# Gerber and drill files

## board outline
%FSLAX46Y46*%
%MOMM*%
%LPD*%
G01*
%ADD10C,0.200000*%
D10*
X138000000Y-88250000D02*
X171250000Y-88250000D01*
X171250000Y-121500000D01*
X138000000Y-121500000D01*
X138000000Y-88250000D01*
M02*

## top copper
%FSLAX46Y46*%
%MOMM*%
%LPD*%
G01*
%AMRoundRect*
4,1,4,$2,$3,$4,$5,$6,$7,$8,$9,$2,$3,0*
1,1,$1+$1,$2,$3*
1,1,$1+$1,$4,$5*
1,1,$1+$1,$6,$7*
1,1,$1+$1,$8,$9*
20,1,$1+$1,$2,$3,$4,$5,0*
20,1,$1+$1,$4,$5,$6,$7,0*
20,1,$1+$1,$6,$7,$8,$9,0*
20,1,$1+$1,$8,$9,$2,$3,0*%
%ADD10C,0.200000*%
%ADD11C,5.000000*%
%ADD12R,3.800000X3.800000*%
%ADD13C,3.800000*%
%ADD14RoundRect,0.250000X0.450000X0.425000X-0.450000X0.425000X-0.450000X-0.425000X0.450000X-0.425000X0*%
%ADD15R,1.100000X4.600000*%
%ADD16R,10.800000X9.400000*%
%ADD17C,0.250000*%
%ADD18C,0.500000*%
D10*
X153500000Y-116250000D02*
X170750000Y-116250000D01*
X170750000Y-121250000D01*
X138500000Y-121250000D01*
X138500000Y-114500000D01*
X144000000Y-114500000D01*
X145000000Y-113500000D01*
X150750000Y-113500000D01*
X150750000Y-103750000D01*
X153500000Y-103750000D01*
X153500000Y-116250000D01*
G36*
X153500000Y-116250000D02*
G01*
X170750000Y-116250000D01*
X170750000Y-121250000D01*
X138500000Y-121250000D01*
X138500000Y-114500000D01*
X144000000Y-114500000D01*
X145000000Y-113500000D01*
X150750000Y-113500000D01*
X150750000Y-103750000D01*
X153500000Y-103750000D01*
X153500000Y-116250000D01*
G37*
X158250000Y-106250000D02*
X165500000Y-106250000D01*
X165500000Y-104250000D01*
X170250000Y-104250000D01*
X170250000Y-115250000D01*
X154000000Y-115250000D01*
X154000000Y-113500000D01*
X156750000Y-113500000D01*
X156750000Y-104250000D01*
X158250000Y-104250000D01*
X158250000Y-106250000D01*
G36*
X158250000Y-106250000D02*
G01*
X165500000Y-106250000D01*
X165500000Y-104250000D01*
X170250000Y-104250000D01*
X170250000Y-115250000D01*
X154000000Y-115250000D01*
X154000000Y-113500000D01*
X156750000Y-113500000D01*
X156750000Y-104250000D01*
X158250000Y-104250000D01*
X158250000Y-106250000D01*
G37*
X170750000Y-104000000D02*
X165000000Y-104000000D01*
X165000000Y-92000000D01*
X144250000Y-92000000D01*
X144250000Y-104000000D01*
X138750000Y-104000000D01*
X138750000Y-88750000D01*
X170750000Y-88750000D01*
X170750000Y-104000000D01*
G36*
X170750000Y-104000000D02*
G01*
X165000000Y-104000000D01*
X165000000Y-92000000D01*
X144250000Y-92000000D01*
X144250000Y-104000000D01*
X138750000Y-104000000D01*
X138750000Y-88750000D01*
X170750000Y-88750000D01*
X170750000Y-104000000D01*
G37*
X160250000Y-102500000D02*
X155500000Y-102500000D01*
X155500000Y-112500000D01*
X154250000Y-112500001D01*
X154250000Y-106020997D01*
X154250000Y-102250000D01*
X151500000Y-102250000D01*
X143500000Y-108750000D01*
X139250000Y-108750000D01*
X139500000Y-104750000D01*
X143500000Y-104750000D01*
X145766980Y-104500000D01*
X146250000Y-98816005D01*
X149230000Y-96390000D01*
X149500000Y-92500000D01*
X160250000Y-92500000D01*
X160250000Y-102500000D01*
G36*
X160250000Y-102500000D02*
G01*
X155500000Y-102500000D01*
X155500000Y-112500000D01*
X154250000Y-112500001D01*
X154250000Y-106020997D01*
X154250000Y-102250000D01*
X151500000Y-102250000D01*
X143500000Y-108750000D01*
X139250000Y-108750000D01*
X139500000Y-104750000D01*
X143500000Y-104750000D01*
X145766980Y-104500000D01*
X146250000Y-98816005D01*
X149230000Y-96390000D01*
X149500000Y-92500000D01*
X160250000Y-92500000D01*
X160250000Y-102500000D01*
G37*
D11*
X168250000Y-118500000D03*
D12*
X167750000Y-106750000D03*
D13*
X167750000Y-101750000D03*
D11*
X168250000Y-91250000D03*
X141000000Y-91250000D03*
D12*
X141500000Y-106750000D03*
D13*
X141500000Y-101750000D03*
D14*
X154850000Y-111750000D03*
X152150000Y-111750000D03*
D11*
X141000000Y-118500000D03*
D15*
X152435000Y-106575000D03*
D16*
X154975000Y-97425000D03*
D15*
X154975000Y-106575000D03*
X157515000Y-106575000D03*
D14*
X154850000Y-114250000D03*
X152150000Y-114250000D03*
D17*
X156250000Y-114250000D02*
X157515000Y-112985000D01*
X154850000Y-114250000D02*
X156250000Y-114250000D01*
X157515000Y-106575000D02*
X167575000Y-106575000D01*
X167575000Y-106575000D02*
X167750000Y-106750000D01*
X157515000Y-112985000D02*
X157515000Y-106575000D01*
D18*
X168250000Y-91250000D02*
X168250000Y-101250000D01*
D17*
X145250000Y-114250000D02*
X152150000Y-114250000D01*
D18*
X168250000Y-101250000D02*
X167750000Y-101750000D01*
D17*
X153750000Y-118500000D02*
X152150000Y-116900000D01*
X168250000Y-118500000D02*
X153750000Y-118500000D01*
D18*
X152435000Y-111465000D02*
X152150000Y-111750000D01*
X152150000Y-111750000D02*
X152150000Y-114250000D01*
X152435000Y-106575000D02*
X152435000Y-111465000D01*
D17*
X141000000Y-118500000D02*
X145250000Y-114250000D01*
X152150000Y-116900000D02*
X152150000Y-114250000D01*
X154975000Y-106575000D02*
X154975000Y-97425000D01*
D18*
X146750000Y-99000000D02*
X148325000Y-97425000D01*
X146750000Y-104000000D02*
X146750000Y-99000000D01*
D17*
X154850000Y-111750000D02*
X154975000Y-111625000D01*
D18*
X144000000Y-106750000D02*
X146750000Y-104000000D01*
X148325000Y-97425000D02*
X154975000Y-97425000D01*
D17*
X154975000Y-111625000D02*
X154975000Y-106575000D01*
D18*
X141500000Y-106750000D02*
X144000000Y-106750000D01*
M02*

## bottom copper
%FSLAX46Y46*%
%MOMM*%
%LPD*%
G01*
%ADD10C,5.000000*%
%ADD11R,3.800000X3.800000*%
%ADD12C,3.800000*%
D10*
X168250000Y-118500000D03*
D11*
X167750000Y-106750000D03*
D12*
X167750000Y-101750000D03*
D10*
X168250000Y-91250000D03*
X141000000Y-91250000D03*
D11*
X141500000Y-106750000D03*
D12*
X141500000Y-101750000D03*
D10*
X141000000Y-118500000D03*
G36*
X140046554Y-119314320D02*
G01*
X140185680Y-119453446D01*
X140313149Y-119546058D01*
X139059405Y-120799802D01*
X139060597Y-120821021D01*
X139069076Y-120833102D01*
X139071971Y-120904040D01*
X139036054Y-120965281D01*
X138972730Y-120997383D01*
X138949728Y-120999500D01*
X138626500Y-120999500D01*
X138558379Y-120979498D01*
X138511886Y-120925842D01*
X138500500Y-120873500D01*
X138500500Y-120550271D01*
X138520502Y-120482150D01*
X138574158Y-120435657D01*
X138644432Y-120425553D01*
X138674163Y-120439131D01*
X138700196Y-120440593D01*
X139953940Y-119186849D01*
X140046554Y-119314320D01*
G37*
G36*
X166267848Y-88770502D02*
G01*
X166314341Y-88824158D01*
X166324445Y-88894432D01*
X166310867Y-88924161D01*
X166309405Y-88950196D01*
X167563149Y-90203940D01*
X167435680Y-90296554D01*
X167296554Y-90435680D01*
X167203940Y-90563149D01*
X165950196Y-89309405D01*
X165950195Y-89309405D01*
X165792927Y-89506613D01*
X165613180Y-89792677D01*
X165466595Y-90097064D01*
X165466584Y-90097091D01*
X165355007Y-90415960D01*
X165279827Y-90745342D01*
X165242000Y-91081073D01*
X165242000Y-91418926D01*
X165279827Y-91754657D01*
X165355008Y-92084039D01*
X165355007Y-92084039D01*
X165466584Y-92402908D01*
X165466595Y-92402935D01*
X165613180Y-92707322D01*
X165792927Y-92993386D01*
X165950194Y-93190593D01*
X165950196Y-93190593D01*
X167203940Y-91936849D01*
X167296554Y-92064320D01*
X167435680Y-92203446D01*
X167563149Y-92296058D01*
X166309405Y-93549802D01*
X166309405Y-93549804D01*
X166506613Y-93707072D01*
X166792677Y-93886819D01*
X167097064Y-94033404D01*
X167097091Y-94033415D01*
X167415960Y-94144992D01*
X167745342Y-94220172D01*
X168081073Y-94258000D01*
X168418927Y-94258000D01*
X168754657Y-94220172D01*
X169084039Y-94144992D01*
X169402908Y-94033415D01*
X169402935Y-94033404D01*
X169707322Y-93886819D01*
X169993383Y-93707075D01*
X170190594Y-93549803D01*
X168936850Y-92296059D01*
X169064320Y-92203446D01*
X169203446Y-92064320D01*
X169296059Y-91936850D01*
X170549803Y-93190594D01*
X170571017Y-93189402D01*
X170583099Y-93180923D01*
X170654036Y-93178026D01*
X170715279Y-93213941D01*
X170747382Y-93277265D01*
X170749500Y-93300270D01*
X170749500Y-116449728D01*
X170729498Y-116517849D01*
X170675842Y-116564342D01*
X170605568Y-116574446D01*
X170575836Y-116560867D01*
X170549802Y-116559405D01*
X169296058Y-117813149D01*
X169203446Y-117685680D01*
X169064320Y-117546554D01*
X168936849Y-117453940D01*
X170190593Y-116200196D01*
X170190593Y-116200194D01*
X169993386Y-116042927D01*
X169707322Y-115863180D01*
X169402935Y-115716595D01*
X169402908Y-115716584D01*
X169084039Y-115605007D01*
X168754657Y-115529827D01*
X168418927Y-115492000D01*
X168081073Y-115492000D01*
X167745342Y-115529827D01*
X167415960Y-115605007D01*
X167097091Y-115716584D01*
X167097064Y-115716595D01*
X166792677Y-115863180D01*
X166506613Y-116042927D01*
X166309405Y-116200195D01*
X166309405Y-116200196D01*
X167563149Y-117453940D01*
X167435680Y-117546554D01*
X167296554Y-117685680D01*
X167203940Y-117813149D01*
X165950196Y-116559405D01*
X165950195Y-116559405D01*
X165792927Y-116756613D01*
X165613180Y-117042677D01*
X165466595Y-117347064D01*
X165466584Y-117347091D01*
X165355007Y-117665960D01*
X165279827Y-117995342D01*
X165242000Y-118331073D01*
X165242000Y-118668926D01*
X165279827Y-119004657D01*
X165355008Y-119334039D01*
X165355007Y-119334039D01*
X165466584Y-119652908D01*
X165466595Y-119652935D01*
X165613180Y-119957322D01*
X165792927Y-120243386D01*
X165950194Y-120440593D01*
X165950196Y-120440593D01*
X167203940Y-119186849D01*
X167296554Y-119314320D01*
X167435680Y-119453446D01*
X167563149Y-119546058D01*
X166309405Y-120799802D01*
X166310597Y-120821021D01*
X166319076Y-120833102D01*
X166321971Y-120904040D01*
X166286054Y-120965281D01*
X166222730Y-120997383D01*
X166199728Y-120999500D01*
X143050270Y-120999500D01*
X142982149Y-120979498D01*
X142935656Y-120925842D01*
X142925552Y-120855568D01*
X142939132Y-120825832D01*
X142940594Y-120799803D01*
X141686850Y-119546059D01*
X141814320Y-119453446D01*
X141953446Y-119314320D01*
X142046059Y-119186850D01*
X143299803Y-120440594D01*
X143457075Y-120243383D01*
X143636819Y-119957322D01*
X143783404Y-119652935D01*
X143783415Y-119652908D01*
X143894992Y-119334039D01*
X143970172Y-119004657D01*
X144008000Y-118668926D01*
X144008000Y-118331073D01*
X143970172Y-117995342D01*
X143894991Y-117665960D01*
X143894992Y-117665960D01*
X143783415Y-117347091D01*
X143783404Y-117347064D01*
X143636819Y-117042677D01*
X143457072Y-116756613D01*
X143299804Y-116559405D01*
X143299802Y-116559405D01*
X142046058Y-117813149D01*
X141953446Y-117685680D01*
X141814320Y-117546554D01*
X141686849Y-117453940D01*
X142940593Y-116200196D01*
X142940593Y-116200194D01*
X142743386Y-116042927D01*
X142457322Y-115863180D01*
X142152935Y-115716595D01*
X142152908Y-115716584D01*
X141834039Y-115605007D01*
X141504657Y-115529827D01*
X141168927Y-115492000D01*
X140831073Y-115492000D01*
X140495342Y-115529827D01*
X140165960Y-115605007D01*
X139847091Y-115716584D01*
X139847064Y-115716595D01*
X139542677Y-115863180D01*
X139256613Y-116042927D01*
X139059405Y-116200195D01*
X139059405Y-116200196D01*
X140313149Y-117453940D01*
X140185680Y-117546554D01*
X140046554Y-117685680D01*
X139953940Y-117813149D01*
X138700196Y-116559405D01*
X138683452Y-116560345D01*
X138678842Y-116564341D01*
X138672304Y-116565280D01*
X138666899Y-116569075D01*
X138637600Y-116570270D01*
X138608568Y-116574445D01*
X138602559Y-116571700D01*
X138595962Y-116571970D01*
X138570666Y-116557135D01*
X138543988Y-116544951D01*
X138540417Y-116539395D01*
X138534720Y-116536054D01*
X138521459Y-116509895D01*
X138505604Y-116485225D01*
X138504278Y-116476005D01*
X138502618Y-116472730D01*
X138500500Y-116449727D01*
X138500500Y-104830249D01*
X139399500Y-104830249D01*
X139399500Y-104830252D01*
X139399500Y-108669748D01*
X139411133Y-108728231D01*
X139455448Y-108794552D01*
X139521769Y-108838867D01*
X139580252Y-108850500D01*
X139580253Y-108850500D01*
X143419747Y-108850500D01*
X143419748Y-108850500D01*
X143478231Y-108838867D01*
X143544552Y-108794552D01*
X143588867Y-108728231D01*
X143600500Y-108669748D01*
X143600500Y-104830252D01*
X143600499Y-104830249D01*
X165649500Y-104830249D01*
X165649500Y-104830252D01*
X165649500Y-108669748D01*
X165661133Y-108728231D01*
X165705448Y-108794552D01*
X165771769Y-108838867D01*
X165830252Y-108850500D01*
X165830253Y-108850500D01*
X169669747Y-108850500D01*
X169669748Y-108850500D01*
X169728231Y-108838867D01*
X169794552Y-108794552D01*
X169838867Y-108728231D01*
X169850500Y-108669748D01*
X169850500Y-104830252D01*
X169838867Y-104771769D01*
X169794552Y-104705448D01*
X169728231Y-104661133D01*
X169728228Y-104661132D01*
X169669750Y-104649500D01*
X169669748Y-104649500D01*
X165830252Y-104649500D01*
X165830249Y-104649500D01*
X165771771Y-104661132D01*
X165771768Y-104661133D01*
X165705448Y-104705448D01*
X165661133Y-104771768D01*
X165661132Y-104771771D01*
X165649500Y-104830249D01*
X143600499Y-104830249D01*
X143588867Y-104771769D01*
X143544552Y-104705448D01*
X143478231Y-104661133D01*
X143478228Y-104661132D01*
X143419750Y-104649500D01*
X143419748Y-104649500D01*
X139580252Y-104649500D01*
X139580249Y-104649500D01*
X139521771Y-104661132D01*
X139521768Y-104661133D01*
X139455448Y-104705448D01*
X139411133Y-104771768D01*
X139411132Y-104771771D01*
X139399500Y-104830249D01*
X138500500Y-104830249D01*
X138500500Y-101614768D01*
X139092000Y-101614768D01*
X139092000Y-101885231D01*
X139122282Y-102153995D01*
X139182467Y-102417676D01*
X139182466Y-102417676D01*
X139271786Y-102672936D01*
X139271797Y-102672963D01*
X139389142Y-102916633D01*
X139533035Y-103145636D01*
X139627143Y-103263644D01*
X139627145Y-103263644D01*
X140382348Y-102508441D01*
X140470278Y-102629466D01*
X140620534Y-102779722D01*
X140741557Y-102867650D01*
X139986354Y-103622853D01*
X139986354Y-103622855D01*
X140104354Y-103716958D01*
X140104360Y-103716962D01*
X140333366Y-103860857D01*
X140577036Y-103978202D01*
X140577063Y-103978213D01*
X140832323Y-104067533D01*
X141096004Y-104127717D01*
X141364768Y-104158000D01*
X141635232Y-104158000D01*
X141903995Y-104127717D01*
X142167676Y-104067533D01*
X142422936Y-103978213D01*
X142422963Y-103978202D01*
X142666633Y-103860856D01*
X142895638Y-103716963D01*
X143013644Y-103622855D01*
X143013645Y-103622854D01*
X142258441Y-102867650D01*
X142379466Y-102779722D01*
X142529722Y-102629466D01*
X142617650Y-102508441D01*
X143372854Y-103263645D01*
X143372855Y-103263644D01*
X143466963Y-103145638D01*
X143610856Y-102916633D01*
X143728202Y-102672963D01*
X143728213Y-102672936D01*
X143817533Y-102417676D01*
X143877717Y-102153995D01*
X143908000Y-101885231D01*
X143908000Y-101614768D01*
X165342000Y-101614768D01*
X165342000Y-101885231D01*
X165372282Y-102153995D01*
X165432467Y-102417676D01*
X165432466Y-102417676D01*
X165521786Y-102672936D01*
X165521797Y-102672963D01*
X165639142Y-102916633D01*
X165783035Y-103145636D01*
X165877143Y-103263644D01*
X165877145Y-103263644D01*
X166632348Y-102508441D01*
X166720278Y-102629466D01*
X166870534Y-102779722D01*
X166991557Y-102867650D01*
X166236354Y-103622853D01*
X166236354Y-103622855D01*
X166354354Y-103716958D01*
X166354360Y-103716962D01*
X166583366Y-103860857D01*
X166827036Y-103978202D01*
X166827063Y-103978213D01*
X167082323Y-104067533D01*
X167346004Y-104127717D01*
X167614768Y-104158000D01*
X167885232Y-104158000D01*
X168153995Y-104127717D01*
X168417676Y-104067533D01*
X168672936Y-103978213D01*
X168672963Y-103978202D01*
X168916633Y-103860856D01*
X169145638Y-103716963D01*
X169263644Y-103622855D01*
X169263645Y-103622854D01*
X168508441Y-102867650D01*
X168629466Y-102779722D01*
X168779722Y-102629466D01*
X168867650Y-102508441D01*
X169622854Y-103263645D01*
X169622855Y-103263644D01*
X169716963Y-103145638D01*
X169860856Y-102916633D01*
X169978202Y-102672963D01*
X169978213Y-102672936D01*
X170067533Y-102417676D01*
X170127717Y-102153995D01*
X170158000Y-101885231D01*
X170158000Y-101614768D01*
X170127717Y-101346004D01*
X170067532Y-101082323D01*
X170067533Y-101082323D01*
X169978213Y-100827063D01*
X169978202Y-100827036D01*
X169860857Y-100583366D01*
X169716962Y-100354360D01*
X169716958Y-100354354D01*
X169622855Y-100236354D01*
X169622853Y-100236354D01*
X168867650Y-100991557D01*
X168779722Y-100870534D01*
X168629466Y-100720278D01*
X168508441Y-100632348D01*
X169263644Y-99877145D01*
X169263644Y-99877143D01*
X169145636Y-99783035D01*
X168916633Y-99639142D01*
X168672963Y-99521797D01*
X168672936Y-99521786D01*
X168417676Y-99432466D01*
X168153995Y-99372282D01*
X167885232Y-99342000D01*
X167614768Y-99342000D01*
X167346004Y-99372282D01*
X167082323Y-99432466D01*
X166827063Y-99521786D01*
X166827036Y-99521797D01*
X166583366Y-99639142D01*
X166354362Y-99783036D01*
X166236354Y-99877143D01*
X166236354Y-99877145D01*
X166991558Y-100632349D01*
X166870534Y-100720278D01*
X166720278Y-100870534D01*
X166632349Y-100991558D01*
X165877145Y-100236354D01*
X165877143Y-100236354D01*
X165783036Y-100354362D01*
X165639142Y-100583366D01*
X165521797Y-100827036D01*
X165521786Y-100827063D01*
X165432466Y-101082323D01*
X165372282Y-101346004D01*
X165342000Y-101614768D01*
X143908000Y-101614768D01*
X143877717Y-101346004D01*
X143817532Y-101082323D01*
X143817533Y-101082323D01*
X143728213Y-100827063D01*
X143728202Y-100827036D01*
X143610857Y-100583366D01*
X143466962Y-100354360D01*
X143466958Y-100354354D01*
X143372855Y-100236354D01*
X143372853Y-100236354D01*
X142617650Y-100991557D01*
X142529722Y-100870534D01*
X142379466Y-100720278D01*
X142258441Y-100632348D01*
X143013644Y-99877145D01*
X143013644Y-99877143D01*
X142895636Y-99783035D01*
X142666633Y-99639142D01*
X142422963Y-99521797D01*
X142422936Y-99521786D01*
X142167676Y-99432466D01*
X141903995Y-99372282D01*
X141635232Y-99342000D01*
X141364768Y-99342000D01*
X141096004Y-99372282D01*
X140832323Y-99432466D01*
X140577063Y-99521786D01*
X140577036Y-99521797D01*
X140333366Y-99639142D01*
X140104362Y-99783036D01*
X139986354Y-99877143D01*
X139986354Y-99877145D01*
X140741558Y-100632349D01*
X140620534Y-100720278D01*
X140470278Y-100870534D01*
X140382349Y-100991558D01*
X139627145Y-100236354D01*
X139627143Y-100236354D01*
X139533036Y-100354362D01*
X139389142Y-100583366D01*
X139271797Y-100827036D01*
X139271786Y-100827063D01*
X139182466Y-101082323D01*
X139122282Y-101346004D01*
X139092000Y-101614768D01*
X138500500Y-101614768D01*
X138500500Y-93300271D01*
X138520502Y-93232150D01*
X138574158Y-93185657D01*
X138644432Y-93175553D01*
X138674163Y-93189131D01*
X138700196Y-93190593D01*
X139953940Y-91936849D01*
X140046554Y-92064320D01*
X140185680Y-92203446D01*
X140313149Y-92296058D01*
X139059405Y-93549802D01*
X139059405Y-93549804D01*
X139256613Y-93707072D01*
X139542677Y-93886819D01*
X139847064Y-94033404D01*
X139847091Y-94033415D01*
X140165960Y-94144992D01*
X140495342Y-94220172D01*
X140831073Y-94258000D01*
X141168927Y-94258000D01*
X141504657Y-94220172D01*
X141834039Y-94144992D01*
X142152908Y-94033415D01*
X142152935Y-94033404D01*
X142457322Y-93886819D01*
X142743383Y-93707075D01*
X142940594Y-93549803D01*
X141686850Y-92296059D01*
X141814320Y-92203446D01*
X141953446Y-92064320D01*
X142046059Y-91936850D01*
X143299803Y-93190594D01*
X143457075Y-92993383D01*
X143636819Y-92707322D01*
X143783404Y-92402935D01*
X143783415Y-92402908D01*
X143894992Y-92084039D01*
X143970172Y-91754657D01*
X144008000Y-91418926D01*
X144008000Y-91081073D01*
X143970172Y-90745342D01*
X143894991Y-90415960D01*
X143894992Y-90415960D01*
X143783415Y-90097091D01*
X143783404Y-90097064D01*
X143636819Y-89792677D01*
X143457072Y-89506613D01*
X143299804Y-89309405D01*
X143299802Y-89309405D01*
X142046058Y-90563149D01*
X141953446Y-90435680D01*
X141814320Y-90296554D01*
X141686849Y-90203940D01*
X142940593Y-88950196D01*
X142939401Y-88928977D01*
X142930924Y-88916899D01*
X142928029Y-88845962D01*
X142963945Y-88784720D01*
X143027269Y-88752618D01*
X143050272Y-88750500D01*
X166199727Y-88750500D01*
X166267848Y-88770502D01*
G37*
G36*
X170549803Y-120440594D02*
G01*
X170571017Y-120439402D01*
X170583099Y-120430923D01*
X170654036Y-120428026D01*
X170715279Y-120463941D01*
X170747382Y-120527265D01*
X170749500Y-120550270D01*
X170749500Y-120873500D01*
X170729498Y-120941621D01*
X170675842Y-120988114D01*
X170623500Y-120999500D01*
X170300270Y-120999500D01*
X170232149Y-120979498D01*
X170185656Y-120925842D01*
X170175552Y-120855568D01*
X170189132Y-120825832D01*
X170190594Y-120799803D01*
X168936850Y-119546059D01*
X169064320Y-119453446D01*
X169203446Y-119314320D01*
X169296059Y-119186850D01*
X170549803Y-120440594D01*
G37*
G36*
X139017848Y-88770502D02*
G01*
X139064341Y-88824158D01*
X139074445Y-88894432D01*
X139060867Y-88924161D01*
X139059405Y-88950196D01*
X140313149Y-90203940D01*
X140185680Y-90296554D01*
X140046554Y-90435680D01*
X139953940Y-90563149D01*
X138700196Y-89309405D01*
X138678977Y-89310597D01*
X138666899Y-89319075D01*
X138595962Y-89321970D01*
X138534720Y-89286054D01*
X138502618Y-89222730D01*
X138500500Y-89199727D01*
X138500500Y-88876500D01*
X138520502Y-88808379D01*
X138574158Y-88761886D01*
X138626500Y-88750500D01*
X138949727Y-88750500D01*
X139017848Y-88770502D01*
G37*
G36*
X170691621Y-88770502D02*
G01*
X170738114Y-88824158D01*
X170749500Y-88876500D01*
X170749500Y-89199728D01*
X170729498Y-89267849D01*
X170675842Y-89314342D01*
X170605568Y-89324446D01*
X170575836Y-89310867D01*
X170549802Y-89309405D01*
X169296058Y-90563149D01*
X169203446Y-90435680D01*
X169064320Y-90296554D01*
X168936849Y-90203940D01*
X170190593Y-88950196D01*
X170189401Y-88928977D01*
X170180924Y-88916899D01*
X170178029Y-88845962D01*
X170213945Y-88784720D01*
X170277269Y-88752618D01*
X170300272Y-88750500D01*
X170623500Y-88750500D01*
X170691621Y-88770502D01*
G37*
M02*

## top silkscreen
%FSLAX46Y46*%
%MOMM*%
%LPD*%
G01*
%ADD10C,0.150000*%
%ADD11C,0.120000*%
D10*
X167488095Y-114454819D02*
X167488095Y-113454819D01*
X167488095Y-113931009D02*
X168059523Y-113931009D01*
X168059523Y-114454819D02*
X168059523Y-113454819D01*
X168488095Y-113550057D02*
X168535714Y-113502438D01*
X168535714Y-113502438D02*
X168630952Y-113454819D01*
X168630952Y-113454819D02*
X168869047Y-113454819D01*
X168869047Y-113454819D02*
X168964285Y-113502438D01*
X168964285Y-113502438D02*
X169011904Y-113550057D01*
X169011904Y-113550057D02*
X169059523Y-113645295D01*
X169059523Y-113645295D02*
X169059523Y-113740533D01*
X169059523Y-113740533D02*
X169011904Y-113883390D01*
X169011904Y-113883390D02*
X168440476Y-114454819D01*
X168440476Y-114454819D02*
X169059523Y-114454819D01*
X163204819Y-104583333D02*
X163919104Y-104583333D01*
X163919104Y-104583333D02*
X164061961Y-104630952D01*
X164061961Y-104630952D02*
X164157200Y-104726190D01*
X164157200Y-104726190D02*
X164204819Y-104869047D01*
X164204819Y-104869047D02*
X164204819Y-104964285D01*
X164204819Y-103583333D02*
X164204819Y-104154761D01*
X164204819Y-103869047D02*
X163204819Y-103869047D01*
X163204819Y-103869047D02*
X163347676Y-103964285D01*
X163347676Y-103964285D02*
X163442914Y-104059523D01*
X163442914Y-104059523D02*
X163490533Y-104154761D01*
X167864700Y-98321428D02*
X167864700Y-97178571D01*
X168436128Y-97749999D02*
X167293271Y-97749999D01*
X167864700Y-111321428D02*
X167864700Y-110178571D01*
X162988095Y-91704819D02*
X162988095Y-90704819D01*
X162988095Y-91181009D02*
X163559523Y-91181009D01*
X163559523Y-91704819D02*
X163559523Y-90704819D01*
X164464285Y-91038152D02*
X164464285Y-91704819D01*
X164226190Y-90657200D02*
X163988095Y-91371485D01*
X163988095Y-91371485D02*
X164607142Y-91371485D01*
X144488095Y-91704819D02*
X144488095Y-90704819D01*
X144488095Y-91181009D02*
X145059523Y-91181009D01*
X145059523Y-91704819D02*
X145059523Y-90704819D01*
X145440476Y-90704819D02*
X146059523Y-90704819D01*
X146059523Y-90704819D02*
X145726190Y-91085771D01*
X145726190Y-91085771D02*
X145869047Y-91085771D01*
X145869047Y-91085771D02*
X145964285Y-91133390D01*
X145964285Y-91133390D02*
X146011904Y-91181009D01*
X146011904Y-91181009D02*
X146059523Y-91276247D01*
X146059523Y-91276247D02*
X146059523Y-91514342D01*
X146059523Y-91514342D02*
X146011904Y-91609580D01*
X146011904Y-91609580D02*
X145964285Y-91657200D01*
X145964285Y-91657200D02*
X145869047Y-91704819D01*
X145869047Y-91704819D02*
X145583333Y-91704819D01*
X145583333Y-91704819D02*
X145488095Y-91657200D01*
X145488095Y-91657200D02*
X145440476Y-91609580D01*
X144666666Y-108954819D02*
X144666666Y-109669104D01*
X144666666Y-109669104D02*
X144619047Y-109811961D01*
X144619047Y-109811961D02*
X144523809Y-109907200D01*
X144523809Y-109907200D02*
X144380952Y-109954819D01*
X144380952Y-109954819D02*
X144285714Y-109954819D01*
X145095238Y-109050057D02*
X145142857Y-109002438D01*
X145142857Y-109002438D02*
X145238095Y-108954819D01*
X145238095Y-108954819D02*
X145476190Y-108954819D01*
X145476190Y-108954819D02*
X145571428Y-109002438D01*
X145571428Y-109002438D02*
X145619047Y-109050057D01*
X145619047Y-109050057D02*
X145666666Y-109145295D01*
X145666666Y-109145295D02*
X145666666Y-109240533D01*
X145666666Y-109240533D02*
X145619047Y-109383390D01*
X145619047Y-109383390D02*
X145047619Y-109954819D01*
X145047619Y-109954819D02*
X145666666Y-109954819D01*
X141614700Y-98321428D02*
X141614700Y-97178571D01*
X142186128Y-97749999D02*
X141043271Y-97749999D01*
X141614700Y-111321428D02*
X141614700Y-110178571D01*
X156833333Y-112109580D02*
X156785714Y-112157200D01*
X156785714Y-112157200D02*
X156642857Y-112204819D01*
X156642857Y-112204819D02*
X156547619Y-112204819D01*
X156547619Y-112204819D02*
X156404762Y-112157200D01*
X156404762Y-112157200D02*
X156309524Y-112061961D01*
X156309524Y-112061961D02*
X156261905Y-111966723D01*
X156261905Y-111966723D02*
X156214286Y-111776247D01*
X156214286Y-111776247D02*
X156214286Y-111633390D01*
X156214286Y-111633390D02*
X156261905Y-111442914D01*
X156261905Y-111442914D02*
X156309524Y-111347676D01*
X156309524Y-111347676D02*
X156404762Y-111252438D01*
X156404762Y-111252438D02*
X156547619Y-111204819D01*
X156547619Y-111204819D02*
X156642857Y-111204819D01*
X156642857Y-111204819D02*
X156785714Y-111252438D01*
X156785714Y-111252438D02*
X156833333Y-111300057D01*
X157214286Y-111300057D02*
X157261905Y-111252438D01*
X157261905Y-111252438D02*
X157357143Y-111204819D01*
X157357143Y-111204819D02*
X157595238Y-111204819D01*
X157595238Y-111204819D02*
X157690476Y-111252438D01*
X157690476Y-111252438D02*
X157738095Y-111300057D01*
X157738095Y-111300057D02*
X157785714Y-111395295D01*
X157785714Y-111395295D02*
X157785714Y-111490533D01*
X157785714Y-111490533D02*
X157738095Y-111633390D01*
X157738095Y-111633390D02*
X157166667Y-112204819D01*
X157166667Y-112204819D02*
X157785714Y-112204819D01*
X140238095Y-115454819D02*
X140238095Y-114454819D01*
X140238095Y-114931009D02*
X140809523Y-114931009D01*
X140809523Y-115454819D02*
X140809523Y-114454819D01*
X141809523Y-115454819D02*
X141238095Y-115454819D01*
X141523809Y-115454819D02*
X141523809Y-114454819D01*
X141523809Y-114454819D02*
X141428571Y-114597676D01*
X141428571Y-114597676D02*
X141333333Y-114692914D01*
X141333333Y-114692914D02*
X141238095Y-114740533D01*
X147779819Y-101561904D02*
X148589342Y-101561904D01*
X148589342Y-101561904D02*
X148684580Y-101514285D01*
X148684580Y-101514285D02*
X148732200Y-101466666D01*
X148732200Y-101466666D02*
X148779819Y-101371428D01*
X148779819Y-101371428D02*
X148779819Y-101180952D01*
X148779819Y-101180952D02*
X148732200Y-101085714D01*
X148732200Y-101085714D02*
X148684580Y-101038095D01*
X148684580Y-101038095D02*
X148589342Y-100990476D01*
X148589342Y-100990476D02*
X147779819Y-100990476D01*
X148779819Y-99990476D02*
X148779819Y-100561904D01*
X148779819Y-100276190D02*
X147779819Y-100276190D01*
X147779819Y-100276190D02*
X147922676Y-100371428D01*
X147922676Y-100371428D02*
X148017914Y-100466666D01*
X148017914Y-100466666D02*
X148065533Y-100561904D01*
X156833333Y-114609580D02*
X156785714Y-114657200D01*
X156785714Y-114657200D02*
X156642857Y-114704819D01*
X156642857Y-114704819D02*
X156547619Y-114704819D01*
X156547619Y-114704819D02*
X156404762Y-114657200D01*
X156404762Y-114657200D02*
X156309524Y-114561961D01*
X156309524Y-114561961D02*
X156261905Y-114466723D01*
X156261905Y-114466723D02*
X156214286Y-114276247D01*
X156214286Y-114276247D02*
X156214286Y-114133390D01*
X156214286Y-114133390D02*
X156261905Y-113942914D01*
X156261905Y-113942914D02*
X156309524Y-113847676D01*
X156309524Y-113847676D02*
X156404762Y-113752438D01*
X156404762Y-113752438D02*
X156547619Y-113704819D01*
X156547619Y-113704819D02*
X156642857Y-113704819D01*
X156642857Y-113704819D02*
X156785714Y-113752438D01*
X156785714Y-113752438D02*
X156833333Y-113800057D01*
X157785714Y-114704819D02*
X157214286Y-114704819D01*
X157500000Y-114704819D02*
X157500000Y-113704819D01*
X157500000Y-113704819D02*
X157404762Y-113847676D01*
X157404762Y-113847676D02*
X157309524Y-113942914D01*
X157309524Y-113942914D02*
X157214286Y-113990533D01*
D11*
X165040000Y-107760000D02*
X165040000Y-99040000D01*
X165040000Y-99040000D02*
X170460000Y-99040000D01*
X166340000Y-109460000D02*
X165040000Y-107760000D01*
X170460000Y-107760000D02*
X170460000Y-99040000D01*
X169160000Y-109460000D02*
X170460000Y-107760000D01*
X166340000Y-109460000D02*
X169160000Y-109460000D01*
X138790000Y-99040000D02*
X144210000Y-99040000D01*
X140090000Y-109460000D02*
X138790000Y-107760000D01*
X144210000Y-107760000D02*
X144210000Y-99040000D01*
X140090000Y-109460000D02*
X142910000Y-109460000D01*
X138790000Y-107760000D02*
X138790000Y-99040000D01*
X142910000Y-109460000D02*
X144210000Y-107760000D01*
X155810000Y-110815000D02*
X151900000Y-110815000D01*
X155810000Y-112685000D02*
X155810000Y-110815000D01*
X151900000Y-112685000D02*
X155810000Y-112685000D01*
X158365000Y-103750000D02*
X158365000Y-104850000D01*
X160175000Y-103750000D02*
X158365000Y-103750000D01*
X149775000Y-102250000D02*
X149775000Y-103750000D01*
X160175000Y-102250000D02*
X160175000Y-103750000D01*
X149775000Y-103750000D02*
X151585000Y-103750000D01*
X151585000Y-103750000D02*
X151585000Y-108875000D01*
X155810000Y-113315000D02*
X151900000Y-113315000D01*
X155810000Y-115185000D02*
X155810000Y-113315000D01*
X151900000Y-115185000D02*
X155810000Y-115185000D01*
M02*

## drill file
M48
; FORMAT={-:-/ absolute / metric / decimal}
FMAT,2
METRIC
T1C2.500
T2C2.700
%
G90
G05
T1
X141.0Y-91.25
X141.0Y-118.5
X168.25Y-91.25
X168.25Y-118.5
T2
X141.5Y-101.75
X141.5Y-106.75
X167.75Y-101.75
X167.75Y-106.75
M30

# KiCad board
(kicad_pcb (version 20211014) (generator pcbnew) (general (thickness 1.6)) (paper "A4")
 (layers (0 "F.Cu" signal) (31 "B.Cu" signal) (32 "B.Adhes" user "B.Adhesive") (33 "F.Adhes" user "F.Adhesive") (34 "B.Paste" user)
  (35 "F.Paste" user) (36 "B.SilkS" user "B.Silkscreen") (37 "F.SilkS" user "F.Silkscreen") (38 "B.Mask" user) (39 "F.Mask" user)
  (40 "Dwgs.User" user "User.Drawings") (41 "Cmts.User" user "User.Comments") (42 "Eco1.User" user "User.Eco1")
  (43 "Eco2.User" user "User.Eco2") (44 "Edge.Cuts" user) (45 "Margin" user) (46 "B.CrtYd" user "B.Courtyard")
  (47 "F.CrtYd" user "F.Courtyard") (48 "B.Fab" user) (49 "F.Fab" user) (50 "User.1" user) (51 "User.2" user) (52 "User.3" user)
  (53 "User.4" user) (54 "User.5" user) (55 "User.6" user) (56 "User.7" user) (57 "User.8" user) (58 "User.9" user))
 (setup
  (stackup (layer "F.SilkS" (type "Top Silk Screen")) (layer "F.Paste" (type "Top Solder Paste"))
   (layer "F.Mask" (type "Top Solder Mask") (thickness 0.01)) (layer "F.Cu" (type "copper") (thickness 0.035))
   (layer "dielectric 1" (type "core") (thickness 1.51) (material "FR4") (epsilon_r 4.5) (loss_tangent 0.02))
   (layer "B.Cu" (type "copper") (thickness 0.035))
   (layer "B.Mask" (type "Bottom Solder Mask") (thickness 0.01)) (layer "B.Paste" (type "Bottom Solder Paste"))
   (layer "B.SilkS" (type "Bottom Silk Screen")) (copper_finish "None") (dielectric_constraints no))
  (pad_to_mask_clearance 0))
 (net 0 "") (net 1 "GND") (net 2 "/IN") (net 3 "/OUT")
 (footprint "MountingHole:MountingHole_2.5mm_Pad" (layer "F.Cu") (at 168.25 118.5)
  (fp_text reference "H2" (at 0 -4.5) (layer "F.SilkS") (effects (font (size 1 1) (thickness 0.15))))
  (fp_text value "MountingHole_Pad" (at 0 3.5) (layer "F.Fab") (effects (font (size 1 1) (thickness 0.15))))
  (pad "1" thru_hole circle (at 0 0) (size 5 5) (drill 2.5) (layers *.Cu *.Mask) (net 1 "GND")))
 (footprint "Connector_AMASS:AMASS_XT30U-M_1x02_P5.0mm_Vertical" (layer "F.Cu") (at 167.75 106.75 90)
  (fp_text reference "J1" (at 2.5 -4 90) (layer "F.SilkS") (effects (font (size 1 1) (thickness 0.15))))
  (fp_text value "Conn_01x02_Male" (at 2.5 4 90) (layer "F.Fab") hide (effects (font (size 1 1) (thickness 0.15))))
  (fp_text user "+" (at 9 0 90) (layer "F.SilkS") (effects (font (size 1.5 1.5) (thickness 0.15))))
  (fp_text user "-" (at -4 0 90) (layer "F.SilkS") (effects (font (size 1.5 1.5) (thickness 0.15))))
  (fp_line (start -1.01 -2.71) (end 7.71 -2.71) (layer "F.SilkS") (width 0.12))
  (fp_line (start 7.71 -2.71) (end 7.71 2.71) (layer "F.SilkS") (width 0.12))
  (fp_line (start -2.71 -1.41) (end -1.01 -2.71) (layer "F.SilkS") (width 0.12))
  (fp_line (start -1.01 2.71) (end 7.71 2.71) (layer "F.SilkS") (width 0.12))
  (fp_line (start -2.71 1.41) (end -1.01 2.71) (layer "F.SilkS") (width 0.12))
  (fp_line (start -2.71 -1.41) (end -2.71 1.41) (layer "F.SilkS") (width 0.12))
  (pad "1" thru_hole rect (at 0 0 90) (size 3.8 3.8) (drill 2.7) (layers *.Cu *.Mask) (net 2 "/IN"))
  (pad "2" thru_hole circle (at 5 0 90) (size 3.8 3.8) (drill 2.7) (layers *.Cu *.Mask) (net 1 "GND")))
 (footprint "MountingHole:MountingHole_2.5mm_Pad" (layer "F.Cu") (at 168.25 91.25)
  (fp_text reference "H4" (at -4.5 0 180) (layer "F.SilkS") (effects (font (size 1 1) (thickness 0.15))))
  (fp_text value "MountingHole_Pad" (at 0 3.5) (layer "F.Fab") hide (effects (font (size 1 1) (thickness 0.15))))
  (pad "1" thru_hole circle (at 0 0) (size 5 5) (drill 2.5) (layers *.Cu *.Mask) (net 1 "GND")))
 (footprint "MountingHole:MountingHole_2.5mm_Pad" (layer "F.Cu") (at 141 91.25)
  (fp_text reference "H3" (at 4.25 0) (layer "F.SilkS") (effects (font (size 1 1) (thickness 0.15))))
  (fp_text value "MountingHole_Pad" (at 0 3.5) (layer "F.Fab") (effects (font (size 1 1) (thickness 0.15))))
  (pad "1" thru_hole circle (at 0 0) (size 5 5) (drill 2.5) (layers *.Cu *.Mask) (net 1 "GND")))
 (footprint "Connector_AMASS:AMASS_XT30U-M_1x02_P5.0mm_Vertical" (layer "F.Cu") (at 141.5 106.75 90)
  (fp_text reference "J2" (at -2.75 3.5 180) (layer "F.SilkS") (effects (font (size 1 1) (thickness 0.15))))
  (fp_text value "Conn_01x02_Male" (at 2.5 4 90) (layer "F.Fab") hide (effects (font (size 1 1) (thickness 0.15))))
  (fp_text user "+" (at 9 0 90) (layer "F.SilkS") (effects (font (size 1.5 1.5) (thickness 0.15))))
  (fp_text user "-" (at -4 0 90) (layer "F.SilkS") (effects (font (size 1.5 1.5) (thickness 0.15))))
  (fp_line (start 7.71 -2.71) (end 7.71 2.71) (layer "F.SilkS") (width 0.12))
  (fp_line (start -2.71 -1.41) (end -1.01 -2.71) (layer "F.SilkS") (width 0.12))
  (fp_line (start -1.01 2.71) (end 7.71 2.71) (layer "F.SilkS") (width 0.12))
  (fp_line (start -2.71 -1.41) (end -2.71 1.41) (layer "F.SilkS") (width 0.12))
  (fp_line (start -1.01 -2.71) (end 7.71 -2.71) (layer "F.SilkS") (width 0.12))
  (fp_line (start -2.71 1.41) (end -1.01 2.71) (layer "F.SilkS") (width 0.12))
  (pad "1" thru_hole rect (at 0 0 90) (size 3.8 3.8) (drill 2.7) (layers *.Cu *.Mask) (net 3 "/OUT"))
  (pad "2" thru_hole circle (at 5 0 90) (size 3.8 3.8) (drill 2.7) (layers *.Cu *.Mask) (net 1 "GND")))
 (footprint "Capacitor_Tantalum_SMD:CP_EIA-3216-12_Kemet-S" (layer "F.Cu") (at 153.5 111.75 180)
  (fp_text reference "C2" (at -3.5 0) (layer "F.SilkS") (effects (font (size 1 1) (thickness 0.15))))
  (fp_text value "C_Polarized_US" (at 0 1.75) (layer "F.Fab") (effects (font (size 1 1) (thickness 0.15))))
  (fp_line (start -2.31 0.935) (end 1.6 0.935) (layer "F.SilkS") (width 0.12))
  (fp_line (start -2.31 -0.935) (end -2.31 0.935) (layer "F.SilkS") (width 0.12))
  (fp_line (start 1.6 -0.935) (end -2.31 -0.935) (layer "F.SilkS") (width 0.12))
  (pad "1" smd roundrect (at -1.35 0 180) (size 1.4 1.35) (layers "F.Cu" "F.Paste" "F.Mask") (roundrect_rratio 0.185185) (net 3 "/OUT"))
  (pad "2" smd roundrect (at 1.35 0 180) (size 1.4 1.35) (layers "F.Cu" "F.Paste" "F.Mask") (roundrect_rratio 0.185185) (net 1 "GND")))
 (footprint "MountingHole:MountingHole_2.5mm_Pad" (layer "F.Cu") (at 141 118.5)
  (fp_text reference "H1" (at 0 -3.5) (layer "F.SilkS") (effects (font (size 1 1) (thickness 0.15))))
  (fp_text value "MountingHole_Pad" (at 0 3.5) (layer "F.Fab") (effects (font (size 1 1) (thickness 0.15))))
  (pad "1" thru_hole circle (at 0 0) (size 5 5) (drill 2.5) (layers *.Cu *.Mask) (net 1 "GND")))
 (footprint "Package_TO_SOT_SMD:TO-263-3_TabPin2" (layer "F.Cu") (at 154.975 100.8 90)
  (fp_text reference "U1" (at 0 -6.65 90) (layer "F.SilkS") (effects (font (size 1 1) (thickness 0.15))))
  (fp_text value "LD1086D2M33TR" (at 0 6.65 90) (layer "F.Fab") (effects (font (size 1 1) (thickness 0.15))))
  (fp_line (start -2.95 3.39) (end -4.05 3.39) (layer "F.SilkS") (width 0.12))
  (fp_line (start -2.95 5.2) (end -2.95 3.39) (layer "F.SilkS") (width 0.12))
  (fp_line (start -1.45 -5.2) (end -2.95 -5.2) (layer "F.SilkS") (width 0.12))
  (fp_line (start -1.45 5.2) (end -2.95 5.2) (layer "F.SilkS") (width 0.12))
  (fp_line (start -2.95 -5.2) (end -2.95 -3.39) (layer "F.SilkS") (width 0.12))
  (fp_line (start -2.95 -3.39) (end -8.075 -3.39) (layer "F.SilkS") (width 0.12))
  (pad "" smd rect (at 5.8 -2.775 90) (size 4.55 5.25) (layers "F.Paste"))
  (pad "" smd rect (at 5.8 2.775 90) (size 4.55 5.25) (layers "F.Paste"))
  (pad "" smd rect (at 0.95 2.775 90) (size 4.55 5.25) (layers "F.Paste"))
  (pad "" smd rect (at 0.95 -2.775 90) (size 4.55 5.25) (layers "F.Paste"))
  (pad "1" smd rect (at -5.775 -2.54 90) (size 4.6 1.1) (layers "F.Cu" "F.Paste" "F.Mask") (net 1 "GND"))
  (pad "2" smd rect (at 3.375 0 90) (size 9.4 10.8) (layers "F.Cu" "F.Mask") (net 3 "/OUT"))
  (pad "2" smd rect (at -5.775 0 90) (size 4.6 1.1) (layers "F.Cu" "F.Paste" "F.Mask") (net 3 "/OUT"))
  (pad "3" smd rect (at -5.775 2.54 90) (size 4.6 1.1) (layers "F.Cu" "F.Paste" "F.Mask") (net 2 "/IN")))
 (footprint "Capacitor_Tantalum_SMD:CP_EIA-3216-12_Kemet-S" (layer "F.Cu") (at 153.5 114.25 180)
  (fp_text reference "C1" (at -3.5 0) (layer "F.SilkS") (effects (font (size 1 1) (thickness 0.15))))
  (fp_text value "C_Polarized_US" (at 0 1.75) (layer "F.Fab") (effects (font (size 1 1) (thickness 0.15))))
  (fp_line (start -2.31 0.935) (end 1.6 0.935) (layer "F.SilkS") (width 0.12))
  (fp_line (start -2.31 -0.935) (end -2.31 0.935) (layer "F.SilkS") (width 0.12))
  (fp_line (start 1.6 -0.935) (end -2.31 -0.935) (layer "F.SilkS") (width 0.12))
  (pad "1" smd roundrect (at -1.35 0 180) (size 1.4 1.35) (layers "F.Cu" "F.Paste" "F.Mask") (roundrect_rratio 0.185185) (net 2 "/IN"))
  (pad "2" smd roundrect (at 1.35 0 180) (size 1.4 1.35) (layers "F.Cu" "F.Paste" "F.Mask") (roundrect_rratio 0.185185) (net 1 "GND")))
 (gr_poly
  (pts (xy 153.5 116.25) (xy 170.75 116.25) (xy 170.75 121.25) (xy 138.5 121.25) (xy 138.5 114.5) (xy 144 114.5) (xy 145 113.5)
   (xy 150.75 113.5) (xy 150.75 103.75) (xy 153.5 103.75))
  (layer "F.Cu") (width 0.2) (fill solid))
 (gr_poly
  (pts (xy 158.25 106.25) (xy 165.5 106.25) (xy 165.5 104.25) (xy 170.25 104.25) (xy 170.25 115.25) (xy 154 115.25) (xy 154 113.5)
   (xy 156.75 113.5) (xy 156.75 104.25) (xy 158.25 104.25))
  (layer "F.Cu") (width 0.2) (fill solid))
 (gr_poly
  (pts (xy 170.75 104) (xy 165 104) (xy 165 92) (xy 144.25 92) (xy 144.25 104) (xy 138.75 104) (xy 138.75 88.75) (xy 170.75 88.75))
  (layer "F.Cu") (width 0.2) (fill solid))
 (gr_poly
  (pts (xy 160.25 102.5) (xy 155.5 102.5) (xy 155.5 112.5) (xy 154.25 112.500001) (xy 154.25 106.020997) (xy 154.25 102.25)
   (xy 151.5 102.25) (xy 143.5 108.75) (xy 139.25 108.75) (xy 139.5 104.75) (xy 143.5 104.75) (xy 145.76698 104.5) (xy 146.25 98.816005)
   (xy 149.23 96.39) (xy 149.5 92.5) (xy 160.25 92.5))
  (layer "F.Cu") (width 0.2) (fill solid))
 (gr_rect (start 138 88.25) (end 171.25 121.5) (layer "Edge.Cuts") (width 0.2) (fill none))
 (segment (start 156.25 114.25) (end 157.515 112.985) (width 0.25) (layer "F.Cu") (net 2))
 (segment (start 154.85 114.25) (end 156.25 114.25) (width 0.25) (layer "F.Cu") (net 2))
 (segment (start 157.515 106.575) (end 167.575 106.575) (width 0.25) (layer "F.Cu") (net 2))
 (segment (start 167.575 106.575) (end 167.75 106.75) (width 0.25) (layer "F.Cu") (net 2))
 (segment (start 157.515 112.985) (end 157.515 106.575) (width 0.25) (layer "F.Cu") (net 2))
 (segment (start 168.25 91.25) (end 168.25 101.25) (width 0.5) (layer "F.Cu") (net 1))
 (segment (start 145.25 114.25) (end 152.15 114.25) (width 0.25) (layer "F.Cu") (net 1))
 (segment (start 168.25 101.25) (end 167.75 101.75) (width 0.5) (layer "F.Cu") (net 1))
 (segment (start 153.75 118.5) (end 152.15 116.9) (width 0.25) (layer "F.Cu") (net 1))
 (segment (start 168.25 118.5) (end 153.75 118.5) (width 0.25) (layer "F.Cu") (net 1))
 (segment (start 152.435 111.465) (end 152.15 111.75) (width 0.5) (layer "F.Cu") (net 1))
 (segment (start 152.15 111.75) (end 152.15 114.25) (width 0.5) (layer "F.Cu") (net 1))
 (segment (start 152.435 106.575) (end 152.435 111.465) (width 0.5) (layer "F.Cu") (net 1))
 (segment (start 141 118.5) (end 145.25 114.25) (width 0.25) (layer "F.Cu") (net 1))
 (segment (start 152.15 116.9) (end 152.15 114.25) (width 0.25) (layer "F.Cu") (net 1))
 (segment (start 154.975 106.575) (end 154.975 97.425) (width 0.25) (layer "F.Cu") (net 3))
 (segment (start 146.75 99) (end 148.325 97.425) (width 0.5) (layer "F.Cu") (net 3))
 (segment (start 146.75 104) (end 146.75 99) (width 0.5) (layer "F.Cu") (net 3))
 (segment (start 154.85 111.75) (end 154.975 111.625) (width 0.25) (layer "F.Cu") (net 3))
 (segment (start 144 106.75) (end 146.75 104) (width 0.5) (layer "F.Cu") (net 3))
 (segment (start 148.325 97.425) (end 154.975 97.425) (width 0.5) (layer "F.Cu") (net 3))
 (segment (start 154.975 111.625) (end 154.975 106.575) (width 0.25) (layer "F.Cu") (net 3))
 (segment (start 141.5 106.75) (end 144 106.75) (width 0.5) (layer "F.Cu") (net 3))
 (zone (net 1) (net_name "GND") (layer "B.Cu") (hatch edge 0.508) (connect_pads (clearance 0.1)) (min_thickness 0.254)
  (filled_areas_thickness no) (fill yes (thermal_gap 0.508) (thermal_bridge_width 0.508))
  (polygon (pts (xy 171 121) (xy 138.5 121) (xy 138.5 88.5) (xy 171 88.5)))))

